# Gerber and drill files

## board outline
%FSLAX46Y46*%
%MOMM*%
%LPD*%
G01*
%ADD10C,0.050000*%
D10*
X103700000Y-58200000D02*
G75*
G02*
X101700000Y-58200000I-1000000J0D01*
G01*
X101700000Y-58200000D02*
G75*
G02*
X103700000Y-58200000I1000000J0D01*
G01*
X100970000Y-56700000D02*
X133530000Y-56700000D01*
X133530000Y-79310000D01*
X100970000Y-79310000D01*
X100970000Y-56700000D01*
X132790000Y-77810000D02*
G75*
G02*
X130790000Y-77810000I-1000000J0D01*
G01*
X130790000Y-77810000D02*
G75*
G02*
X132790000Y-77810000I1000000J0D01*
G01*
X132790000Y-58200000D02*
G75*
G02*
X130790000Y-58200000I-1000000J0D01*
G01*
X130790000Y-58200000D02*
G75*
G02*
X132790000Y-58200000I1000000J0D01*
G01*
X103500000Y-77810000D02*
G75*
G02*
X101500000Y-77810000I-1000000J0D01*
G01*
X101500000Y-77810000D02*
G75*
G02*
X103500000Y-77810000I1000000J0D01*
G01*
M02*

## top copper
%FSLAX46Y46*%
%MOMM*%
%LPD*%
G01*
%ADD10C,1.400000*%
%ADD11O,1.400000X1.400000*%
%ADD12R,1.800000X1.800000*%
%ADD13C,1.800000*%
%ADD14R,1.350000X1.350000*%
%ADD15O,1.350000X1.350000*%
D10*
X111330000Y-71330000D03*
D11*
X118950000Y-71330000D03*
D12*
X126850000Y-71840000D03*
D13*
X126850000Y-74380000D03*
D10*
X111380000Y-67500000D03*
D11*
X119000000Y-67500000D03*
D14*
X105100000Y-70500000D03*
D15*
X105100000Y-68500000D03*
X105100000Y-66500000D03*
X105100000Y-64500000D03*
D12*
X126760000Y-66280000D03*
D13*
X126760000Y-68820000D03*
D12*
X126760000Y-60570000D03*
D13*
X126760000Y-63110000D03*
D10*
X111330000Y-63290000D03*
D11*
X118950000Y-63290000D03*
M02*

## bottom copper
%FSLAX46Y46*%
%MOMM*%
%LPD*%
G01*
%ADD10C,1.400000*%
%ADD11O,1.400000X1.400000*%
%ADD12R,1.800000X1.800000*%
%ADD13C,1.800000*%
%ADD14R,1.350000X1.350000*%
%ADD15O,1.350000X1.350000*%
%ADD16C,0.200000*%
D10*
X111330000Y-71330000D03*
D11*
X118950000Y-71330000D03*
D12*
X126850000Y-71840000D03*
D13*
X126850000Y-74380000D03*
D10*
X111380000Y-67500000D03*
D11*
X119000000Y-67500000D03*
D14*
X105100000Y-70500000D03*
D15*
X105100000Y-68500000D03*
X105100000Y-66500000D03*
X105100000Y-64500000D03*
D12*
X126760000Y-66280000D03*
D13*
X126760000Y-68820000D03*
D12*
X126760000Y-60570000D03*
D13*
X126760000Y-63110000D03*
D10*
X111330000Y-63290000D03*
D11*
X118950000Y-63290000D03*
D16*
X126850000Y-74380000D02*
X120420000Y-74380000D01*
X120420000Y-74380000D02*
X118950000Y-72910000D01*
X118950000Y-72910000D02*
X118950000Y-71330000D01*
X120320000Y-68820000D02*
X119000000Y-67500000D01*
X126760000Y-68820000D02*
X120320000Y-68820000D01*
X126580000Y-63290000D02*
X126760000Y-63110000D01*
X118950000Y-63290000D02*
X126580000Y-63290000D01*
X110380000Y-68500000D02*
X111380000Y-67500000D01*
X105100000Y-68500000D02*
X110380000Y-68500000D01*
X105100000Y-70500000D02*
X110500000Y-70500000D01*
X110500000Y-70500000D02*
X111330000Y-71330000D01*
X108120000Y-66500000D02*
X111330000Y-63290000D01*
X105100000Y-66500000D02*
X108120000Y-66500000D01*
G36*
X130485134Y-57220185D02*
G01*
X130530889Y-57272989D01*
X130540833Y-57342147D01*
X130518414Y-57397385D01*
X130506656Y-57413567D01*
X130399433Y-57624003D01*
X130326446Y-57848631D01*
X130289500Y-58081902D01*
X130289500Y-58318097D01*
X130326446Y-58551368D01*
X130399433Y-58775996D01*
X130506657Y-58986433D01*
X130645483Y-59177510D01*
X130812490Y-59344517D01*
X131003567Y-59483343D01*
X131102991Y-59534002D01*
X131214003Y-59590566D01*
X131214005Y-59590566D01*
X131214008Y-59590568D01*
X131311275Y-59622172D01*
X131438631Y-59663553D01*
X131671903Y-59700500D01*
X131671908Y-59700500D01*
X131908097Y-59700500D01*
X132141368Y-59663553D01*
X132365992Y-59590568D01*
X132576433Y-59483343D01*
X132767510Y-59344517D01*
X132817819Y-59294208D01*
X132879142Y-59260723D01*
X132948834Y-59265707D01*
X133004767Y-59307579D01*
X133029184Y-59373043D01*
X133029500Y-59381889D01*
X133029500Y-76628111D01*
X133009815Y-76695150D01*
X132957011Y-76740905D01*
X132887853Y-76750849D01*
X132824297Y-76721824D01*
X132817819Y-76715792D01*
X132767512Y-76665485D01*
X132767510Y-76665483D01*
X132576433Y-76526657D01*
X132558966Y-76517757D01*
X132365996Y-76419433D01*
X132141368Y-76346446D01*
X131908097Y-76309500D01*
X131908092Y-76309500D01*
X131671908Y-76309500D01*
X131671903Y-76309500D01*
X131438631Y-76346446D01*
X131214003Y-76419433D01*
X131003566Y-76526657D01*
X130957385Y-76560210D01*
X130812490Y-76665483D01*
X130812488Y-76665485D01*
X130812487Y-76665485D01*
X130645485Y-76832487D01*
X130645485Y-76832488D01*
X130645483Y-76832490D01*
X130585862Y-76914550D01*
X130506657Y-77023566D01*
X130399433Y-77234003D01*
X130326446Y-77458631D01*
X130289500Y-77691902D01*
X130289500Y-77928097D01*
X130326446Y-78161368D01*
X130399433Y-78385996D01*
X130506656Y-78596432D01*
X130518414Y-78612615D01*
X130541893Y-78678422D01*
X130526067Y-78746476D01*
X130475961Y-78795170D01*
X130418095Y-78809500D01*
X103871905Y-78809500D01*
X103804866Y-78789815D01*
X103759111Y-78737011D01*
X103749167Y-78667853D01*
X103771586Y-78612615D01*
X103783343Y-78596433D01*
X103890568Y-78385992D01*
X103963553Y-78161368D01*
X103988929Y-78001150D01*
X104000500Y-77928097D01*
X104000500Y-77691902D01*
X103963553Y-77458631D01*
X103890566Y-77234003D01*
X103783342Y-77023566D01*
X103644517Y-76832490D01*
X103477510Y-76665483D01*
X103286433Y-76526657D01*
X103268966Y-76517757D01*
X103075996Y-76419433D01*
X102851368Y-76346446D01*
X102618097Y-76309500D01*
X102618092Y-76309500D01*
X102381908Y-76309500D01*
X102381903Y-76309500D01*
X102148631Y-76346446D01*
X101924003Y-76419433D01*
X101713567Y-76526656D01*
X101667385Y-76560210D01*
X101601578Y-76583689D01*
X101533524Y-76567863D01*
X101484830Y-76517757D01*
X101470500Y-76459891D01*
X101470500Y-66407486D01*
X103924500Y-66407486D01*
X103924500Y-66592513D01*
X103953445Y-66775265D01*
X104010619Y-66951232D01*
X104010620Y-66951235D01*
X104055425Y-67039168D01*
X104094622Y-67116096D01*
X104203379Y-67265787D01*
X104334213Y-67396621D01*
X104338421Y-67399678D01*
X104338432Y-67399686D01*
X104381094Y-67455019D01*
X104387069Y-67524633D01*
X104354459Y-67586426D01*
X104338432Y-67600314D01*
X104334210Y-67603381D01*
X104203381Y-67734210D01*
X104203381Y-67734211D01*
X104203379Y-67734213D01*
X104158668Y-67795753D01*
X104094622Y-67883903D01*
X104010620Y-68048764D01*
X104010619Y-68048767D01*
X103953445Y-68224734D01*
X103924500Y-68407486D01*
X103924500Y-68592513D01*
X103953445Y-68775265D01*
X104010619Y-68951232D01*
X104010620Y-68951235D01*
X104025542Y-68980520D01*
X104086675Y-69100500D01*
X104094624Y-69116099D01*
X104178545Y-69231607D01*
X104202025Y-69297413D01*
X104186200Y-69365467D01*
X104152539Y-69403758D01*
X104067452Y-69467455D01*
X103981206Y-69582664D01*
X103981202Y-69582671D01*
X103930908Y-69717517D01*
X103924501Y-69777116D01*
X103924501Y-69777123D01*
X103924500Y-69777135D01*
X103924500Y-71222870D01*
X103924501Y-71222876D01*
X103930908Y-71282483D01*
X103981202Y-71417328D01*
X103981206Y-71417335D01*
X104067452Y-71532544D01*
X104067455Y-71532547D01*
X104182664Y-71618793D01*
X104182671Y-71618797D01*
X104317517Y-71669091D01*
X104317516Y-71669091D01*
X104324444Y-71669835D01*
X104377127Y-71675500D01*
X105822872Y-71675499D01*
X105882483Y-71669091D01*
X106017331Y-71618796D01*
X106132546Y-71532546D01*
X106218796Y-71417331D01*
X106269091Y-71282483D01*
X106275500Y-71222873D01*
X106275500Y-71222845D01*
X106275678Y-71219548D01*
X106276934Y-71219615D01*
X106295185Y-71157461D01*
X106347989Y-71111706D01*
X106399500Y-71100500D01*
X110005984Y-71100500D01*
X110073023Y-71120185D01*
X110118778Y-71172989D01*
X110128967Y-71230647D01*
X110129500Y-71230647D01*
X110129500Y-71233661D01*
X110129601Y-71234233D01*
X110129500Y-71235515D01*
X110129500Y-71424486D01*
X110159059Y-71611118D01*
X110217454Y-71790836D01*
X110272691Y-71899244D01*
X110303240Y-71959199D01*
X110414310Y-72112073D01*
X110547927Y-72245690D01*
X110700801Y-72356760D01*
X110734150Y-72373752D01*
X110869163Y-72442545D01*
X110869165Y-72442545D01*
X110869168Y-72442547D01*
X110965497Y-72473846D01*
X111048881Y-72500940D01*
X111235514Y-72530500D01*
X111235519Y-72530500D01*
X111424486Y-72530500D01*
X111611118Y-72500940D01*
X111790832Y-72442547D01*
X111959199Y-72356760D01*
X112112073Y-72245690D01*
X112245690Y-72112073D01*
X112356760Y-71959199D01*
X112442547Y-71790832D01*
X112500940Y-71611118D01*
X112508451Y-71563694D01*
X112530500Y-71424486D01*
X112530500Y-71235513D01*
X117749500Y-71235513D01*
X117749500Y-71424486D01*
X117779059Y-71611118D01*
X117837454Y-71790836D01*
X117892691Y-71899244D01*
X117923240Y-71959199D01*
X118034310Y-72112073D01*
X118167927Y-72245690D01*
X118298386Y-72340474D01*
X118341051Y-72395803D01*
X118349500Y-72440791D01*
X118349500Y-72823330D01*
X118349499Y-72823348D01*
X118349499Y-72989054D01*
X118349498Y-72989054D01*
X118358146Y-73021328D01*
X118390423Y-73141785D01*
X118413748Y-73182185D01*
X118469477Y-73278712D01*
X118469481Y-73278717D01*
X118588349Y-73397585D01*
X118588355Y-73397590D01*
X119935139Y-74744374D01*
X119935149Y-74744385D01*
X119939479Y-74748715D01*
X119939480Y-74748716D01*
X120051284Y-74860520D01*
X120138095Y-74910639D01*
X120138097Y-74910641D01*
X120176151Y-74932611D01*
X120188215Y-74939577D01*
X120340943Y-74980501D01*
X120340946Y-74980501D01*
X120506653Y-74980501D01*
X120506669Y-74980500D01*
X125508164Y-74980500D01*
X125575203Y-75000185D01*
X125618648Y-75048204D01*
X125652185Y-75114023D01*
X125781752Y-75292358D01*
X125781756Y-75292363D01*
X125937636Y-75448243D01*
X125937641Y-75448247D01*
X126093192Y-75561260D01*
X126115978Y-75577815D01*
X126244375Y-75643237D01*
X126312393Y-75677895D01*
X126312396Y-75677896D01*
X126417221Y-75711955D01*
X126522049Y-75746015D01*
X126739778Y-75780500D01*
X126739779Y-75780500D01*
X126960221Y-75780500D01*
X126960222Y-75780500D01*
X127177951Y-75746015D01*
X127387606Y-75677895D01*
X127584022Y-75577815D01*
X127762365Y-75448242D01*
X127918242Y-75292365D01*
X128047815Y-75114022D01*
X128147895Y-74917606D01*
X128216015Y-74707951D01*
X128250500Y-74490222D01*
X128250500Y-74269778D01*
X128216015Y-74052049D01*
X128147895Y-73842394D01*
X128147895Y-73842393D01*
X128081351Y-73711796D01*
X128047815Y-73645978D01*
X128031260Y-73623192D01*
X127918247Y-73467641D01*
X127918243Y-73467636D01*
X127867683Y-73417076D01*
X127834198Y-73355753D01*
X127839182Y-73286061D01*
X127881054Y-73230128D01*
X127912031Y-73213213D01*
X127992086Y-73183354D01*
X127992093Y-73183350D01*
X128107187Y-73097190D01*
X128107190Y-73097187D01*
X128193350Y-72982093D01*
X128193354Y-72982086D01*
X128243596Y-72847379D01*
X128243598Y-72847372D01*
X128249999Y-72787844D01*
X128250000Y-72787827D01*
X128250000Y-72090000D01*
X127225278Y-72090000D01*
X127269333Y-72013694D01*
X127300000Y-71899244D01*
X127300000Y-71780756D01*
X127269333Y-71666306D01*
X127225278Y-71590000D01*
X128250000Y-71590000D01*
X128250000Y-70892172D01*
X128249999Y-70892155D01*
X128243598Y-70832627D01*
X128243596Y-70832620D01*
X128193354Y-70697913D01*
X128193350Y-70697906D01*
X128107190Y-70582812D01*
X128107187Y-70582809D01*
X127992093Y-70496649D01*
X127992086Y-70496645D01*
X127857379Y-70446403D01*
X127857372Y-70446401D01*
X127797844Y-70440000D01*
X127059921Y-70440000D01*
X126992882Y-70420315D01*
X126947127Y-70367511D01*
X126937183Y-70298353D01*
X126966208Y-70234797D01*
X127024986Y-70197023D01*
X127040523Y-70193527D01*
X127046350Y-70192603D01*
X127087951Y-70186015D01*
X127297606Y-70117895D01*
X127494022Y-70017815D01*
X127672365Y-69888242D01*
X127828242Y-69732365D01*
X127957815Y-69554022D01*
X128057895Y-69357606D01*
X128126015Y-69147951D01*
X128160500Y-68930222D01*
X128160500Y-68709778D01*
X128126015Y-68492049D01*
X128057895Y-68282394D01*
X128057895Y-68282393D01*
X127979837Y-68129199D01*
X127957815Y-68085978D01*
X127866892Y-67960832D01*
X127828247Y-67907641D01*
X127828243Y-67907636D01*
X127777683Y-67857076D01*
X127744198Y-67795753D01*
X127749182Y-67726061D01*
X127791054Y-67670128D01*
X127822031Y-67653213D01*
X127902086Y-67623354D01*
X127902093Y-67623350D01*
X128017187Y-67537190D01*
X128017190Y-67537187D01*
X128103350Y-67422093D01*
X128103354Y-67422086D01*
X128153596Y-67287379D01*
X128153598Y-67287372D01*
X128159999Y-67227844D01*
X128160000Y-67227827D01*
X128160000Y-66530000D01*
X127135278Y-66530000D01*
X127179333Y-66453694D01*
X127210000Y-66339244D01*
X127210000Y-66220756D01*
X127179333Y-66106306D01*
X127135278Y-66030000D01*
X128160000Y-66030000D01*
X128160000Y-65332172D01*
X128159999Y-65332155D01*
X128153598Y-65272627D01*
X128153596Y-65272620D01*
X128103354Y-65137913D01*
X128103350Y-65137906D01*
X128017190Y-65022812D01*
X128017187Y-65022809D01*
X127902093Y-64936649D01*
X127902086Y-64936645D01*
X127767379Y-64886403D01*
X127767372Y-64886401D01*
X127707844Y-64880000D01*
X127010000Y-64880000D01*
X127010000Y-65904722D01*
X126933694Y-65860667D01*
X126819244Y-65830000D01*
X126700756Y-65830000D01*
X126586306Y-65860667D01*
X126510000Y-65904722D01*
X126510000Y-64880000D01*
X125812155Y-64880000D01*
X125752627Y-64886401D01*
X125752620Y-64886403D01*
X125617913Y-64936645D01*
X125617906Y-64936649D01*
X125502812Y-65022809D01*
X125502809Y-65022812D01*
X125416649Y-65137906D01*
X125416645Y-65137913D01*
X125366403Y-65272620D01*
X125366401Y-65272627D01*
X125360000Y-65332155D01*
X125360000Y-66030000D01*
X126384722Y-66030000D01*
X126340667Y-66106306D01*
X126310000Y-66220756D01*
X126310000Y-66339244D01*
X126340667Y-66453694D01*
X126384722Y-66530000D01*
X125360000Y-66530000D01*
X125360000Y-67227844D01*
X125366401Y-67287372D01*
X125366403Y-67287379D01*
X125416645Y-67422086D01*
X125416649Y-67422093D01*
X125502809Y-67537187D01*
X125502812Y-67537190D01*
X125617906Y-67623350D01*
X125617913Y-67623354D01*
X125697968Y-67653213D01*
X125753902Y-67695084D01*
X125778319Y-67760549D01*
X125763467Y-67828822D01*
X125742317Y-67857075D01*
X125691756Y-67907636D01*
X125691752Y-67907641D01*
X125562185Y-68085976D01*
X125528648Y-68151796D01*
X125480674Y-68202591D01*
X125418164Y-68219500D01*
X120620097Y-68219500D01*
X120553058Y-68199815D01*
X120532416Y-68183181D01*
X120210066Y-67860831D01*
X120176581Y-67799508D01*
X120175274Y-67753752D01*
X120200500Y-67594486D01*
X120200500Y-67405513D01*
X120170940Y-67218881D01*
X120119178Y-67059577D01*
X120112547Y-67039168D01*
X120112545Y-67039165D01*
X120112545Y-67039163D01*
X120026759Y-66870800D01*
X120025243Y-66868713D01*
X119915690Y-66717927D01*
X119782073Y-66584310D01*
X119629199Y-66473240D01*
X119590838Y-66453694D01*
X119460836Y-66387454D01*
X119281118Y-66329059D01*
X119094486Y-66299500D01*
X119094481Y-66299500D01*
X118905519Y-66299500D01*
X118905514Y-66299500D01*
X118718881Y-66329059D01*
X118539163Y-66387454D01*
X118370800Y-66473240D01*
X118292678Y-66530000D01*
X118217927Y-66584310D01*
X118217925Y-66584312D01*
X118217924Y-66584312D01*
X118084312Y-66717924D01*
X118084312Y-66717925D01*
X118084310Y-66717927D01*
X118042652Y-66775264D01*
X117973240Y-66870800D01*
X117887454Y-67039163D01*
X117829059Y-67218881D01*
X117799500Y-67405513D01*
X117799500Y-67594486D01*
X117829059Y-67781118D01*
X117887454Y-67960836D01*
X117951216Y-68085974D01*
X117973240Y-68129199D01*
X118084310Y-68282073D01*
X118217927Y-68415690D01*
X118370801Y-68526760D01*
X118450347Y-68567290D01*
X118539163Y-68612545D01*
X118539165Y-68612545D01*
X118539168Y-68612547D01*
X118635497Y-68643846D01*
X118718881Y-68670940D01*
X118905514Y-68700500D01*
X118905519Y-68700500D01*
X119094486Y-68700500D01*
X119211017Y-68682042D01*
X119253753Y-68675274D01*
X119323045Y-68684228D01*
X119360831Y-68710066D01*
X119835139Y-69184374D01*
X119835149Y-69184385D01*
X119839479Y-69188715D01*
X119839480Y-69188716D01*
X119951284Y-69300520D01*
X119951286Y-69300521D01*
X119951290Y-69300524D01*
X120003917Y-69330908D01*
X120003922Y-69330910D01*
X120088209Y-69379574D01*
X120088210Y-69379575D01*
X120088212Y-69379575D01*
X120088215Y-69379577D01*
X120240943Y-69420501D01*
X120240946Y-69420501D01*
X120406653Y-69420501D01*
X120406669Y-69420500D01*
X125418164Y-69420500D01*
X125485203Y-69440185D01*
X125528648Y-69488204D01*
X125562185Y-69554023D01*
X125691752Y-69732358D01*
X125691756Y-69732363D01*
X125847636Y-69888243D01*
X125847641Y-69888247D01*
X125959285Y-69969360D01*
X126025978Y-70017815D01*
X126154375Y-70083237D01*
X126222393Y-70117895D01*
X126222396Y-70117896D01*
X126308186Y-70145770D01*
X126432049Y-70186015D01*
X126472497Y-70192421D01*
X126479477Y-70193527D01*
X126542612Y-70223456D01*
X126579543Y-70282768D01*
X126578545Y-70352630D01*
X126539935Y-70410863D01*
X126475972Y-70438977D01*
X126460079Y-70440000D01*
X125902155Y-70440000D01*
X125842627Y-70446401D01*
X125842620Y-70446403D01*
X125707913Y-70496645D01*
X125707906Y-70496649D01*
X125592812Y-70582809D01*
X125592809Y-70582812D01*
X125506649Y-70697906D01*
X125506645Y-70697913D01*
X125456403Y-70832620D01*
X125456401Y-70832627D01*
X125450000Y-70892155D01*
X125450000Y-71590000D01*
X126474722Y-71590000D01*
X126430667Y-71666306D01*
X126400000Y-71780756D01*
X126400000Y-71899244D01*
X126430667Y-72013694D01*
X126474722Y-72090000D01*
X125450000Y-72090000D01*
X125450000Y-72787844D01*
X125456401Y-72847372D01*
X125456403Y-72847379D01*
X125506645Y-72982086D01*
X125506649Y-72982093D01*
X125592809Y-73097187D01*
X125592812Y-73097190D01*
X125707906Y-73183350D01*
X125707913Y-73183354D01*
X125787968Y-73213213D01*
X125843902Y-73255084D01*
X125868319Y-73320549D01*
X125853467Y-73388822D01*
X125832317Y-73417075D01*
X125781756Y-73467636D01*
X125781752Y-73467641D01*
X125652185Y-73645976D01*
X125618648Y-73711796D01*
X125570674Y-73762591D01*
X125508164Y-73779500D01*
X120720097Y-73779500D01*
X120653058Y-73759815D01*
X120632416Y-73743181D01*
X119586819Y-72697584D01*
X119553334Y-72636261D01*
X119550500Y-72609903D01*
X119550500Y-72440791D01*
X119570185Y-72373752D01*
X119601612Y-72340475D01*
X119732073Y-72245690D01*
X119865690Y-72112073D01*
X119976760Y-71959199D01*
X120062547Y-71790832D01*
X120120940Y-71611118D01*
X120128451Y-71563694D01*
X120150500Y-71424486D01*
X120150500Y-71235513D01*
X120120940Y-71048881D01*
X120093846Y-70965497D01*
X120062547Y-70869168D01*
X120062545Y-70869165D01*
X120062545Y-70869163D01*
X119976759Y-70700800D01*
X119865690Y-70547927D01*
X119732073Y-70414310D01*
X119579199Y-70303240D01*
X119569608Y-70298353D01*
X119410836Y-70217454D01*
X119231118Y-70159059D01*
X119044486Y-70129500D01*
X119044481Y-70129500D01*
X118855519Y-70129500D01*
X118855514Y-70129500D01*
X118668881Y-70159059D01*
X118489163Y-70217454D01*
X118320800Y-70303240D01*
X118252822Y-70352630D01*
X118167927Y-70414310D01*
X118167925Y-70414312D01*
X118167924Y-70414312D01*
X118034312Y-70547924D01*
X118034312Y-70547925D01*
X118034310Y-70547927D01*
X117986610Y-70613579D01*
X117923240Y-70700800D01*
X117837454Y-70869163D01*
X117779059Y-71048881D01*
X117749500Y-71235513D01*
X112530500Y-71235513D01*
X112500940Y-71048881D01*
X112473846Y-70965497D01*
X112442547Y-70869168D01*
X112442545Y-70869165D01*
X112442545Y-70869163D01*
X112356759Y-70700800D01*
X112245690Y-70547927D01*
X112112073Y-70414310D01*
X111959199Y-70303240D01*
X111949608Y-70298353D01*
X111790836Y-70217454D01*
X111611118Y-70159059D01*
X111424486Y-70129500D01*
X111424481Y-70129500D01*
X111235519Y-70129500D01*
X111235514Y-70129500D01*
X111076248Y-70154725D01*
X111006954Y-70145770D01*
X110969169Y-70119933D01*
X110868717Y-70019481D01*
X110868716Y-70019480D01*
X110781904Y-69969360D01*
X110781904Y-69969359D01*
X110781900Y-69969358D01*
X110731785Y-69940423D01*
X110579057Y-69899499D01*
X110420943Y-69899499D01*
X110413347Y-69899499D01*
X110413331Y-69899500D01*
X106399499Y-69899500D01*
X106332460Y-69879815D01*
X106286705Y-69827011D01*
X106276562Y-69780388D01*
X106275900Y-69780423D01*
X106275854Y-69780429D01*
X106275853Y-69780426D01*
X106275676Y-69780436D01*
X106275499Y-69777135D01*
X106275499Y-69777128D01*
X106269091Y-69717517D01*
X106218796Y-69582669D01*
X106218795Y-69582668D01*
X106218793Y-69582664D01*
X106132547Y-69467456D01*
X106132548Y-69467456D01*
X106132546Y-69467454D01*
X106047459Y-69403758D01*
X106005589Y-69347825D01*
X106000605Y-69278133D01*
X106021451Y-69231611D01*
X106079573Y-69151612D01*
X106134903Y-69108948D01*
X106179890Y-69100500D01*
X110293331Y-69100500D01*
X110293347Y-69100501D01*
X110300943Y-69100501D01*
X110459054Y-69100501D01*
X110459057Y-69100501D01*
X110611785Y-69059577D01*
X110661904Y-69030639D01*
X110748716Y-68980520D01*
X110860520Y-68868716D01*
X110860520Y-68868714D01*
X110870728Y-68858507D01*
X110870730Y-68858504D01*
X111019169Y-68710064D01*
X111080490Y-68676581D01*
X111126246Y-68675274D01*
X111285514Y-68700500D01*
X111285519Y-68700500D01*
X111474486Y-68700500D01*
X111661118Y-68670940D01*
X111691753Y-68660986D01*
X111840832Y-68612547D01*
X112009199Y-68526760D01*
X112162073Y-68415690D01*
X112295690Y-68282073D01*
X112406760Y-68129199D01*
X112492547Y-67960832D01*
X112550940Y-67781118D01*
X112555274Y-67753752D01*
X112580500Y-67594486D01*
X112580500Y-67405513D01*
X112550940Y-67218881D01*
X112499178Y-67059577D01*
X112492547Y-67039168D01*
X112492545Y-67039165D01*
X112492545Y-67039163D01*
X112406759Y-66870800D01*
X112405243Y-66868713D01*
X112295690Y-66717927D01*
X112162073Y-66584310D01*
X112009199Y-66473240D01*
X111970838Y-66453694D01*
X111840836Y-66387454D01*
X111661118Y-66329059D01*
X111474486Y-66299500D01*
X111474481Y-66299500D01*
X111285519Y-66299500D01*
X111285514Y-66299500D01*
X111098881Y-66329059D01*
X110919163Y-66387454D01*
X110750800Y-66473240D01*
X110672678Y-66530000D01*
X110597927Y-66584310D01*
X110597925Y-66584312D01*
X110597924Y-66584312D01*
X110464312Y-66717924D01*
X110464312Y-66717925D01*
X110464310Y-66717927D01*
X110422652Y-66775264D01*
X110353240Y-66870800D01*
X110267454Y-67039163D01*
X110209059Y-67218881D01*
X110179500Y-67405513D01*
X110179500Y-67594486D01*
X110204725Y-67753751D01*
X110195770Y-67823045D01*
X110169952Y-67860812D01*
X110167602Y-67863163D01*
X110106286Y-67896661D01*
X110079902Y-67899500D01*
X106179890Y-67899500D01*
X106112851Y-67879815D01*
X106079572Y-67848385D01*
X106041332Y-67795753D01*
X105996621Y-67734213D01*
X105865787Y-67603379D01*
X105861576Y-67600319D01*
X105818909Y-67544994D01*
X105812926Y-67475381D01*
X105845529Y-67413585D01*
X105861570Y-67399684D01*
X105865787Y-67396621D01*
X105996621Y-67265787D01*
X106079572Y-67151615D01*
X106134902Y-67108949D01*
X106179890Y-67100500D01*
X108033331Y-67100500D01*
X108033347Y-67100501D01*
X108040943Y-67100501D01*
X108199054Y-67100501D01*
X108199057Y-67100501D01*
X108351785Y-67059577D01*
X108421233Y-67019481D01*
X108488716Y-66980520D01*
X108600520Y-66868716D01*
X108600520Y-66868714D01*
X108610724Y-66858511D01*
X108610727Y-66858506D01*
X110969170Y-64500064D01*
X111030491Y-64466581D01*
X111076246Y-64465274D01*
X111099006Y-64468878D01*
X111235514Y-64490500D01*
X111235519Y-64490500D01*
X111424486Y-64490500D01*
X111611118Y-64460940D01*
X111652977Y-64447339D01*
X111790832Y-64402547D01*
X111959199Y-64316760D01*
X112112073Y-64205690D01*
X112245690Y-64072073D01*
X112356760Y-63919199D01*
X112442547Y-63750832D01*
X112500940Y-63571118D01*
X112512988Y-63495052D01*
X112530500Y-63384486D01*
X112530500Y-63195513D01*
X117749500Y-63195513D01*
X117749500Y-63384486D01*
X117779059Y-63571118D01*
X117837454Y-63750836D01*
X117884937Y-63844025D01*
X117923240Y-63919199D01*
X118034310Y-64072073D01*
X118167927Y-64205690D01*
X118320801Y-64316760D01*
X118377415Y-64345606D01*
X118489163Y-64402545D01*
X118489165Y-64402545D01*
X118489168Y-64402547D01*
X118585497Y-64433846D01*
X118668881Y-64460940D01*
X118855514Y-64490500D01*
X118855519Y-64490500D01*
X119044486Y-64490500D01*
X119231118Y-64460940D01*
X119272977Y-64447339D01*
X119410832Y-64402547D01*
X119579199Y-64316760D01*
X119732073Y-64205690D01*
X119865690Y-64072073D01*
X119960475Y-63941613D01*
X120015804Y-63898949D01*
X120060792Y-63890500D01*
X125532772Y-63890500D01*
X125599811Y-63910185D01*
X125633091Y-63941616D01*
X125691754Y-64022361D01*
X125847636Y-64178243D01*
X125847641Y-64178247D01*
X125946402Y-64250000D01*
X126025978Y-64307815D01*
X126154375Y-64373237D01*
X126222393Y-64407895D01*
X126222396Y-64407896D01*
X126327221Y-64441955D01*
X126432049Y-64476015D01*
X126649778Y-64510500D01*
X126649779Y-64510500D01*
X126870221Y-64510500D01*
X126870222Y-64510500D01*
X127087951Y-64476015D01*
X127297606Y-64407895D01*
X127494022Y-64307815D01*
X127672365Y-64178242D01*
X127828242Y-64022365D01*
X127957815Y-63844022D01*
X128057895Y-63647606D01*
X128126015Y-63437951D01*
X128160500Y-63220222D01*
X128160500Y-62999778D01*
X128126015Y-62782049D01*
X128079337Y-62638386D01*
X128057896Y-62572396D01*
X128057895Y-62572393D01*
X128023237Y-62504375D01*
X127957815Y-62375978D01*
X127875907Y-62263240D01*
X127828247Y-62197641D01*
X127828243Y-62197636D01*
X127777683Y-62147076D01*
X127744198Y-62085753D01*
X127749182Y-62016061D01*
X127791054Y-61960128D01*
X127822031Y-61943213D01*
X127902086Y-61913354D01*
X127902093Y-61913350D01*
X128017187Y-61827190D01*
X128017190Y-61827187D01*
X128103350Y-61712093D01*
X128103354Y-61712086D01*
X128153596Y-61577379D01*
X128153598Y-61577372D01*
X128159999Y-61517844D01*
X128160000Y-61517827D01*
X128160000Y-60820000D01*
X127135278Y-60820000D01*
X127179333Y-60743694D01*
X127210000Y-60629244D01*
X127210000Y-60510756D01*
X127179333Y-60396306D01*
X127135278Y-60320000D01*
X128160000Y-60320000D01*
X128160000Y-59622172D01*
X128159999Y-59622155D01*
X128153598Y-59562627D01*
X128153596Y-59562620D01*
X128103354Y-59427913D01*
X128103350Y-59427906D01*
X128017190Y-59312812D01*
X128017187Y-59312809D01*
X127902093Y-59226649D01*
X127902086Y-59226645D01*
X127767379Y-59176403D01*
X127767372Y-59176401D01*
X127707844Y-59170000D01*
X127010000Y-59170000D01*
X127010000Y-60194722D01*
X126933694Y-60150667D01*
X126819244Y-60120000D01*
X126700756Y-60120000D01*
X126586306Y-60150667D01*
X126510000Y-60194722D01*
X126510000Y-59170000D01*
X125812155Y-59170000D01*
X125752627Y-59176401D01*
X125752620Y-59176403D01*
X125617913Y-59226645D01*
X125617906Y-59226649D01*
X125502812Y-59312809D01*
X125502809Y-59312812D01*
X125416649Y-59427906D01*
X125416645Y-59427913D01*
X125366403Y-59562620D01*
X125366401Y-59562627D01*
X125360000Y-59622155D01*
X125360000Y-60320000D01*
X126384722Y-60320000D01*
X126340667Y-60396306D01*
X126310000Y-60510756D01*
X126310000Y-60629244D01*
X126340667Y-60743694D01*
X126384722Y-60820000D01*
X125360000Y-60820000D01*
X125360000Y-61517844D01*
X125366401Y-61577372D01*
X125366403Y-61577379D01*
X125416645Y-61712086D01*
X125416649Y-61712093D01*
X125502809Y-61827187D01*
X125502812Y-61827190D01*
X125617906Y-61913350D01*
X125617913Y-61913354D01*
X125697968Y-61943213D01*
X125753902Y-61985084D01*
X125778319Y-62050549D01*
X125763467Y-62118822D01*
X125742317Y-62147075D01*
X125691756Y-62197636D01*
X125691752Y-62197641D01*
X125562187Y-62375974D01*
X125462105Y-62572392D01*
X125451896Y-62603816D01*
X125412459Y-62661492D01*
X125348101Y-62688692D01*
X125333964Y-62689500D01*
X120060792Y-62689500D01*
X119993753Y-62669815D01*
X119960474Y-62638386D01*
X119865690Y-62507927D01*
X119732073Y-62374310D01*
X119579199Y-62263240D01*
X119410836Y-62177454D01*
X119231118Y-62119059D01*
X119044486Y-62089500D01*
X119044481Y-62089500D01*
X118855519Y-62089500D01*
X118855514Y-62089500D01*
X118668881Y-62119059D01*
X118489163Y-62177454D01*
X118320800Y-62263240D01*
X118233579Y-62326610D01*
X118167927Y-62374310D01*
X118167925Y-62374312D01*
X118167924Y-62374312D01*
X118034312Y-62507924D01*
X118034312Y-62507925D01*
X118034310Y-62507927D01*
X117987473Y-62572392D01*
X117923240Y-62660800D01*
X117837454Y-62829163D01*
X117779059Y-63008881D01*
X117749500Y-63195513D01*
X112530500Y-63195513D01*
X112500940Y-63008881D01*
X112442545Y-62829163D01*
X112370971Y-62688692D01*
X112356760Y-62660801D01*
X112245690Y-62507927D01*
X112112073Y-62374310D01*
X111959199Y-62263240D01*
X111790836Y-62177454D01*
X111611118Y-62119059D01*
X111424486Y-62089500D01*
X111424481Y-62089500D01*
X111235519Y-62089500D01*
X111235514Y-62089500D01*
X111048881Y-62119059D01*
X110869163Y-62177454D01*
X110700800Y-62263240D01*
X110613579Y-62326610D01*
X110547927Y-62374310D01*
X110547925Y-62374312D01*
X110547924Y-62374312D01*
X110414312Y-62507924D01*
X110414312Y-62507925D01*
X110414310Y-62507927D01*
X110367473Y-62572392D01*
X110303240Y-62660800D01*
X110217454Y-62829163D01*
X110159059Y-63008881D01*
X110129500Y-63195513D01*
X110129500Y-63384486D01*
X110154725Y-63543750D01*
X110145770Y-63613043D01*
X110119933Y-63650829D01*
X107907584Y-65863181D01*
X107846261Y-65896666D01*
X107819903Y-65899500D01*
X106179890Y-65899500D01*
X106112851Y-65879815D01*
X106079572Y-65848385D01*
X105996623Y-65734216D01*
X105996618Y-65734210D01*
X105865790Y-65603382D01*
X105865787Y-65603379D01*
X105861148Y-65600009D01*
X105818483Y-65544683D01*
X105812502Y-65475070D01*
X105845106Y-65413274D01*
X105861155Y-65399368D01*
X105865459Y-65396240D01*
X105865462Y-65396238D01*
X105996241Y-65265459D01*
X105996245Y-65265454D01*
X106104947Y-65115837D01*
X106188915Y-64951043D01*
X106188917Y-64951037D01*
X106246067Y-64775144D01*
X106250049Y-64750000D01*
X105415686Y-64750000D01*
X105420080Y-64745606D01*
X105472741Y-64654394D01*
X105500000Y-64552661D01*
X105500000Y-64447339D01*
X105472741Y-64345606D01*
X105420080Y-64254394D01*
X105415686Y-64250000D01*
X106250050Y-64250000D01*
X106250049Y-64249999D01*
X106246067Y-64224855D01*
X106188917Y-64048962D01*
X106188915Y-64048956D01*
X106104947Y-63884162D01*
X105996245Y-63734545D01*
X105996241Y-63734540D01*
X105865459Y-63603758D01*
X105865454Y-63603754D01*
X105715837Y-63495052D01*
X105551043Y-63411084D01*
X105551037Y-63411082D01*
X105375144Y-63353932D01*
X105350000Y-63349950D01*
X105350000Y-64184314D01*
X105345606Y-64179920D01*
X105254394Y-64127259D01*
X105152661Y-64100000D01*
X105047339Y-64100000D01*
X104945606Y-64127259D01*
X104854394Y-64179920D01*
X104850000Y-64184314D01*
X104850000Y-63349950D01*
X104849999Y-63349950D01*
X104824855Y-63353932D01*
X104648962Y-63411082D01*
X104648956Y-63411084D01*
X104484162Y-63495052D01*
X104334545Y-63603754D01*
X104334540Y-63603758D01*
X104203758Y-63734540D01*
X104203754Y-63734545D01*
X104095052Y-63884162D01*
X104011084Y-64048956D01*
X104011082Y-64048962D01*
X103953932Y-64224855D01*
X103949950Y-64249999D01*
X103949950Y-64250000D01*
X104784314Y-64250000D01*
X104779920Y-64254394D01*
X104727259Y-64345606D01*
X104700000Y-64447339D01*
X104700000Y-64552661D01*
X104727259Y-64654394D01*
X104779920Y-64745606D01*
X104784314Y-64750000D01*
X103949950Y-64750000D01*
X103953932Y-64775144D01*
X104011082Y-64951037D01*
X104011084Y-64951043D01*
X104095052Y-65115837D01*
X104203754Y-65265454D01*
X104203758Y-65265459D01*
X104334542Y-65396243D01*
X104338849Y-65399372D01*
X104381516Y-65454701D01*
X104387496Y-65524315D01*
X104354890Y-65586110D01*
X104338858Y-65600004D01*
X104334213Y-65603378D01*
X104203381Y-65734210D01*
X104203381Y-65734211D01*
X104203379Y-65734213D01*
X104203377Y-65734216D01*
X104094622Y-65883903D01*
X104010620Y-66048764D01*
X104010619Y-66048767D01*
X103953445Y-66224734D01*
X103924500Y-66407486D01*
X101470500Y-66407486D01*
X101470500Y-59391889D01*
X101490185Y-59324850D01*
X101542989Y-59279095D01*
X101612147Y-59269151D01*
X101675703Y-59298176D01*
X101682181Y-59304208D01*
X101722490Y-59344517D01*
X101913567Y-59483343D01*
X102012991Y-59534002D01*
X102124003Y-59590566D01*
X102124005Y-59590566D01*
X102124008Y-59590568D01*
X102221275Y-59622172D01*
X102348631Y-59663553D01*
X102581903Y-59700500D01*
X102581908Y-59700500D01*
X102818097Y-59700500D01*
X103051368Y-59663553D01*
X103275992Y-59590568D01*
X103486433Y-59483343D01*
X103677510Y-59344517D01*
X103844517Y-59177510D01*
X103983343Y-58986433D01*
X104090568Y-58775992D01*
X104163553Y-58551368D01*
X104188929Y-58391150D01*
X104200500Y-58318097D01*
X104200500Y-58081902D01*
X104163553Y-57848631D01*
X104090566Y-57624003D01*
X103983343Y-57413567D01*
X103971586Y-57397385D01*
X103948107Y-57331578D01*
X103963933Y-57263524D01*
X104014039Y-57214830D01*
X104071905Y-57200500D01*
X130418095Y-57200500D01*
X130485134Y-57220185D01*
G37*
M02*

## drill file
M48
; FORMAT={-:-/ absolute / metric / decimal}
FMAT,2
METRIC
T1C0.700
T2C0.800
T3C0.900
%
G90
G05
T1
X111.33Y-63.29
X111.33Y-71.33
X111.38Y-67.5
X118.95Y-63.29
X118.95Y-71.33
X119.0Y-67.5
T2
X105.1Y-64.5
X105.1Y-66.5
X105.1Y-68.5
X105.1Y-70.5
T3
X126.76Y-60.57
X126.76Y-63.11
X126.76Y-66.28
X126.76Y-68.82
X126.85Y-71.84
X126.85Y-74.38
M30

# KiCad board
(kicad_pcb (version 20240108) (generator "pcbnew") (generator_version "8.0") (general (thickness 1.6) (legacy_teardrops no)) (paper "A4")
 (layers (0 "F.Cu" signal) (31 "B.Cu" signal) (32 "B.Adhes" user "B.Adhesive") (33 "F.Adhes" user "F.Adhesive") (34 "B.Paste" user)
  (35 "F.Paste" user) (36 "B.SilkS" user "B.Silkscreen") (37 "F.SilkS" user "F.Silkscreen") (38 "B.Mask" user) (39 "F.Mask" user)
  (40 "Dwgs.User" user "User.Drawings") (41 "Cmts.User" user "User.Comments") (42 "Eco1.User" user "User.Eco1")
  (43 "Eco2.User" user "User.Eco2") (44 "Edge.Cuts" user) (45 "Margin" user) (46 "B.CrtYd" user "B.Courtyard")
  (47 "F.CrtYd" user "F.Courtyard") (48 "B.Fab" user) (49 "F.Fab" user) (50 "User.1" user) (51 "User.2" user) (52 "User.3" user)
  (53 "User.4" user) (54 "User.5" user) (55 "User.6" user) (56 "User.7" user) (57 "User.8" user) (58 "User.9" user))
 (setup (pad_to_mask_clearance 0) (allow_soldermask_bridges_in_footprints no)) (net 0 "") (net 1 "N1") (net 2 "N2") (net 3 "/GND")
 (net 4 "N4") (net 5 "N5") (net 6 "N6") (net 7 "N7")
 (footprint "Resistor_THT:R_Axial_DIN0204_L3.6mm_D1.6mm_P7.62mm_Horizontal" (layer "F.Cu") (at 111.33 71.33)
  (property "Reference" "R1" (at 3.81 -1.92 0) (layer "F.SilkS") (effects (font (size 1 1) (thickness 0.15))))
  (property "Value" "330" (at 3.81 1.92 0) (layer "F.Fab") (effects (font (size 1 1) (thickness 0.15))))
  (pad "1" thru_hole circle (at 0 0) (size 1.4 1.4) (drill 0.7) (layers "*.Cu" "*.Mask") (remove_unused_layers no) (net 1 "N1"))
  (pad "2" thru_hole oval (at 7.62 0) (size 1.4 1.4) (drill 0.7) (layers "*.Cu" "*.Mask") (remove_unused_layers no) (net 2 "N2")))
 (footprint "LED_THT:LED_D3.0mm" (layer "F.Cu") (at 126.85 71.84 -90)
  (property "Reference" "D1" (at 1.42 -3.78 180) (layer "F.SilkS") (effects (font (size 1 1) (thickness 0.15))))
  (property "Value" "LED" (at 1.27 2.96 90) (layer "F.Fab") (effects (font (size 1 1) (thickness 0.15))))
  (pad "1" thru_hole rect (at 0 0 270) (size 1.8 1.8) (drill 0.9) (layers "*.Cu" "*.Mask") (remove_unused_layers no) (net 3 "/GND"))
  (pad "2" thru_hole circle (at 2.54 0 270) (size 1.8 1.8) (drill 0.9) (layers "*.Cu" "*.Mask") (remove_unused_layers no) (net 2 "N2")))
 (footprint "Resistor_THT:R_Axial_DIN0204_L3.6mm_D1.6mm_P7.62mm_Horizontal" (layer "F.Cu") (at 111.38 67.5)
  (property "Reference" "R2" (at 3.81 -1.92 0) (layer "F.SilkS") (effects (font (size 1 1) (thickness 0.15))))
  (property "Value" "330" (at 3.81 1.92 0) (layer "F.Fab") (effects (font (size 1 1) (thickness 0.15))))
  (pad "1" thru_hole circle (at 0 0) (size 1.4 1.4) (drill 0.7) (layers "*.Cu" "*.Mask") (remove_unused_layers no) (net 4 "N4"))
  (pad "2" thru_hole oval (at 7.62 0) (size 1.4 1.4) (drill 0.7) (layers "*.Cu" "*.Mask") (remove_unused_layers no) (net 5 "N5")))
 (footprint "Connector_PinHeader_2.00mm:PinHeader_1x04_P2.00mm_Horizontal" (layer "F.Cu") (at 105.1 70.5 180)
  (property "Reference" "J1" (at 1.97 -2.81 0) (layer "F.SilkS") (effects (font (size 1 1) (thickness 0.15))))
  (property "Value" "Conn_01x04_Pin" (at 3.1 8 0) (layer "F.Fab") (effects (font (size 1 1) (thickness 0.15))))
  (pad "1" thru_hole rect (at 0 0 180) (size 1.35 1.35) (drill 0.8) (layers "*.Cu" "*.Mask") (remove_unused_layers no) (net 1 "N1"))
  (pad "2" thru_hole oval (at 0 2 180) (size 1.35 1.35) (drill 0.8) (layers "*.Cu" "*.Mask") (remove_unused_layers no) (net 4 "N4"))
  (pad "3" thru_hole oval (at 0 4 180) (size 1.35 1.35) (drill 0.8) (layers "*.Cu" "*.Mask") (remove_unused_layers no) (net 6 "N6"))
  (pad "4" thru_hole oval (at 0 6 180) (size 1.35 1.35) (drill 0.8) (layers "*.Cu" "*.Mask") (remove_unused_layers no) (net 3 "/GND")))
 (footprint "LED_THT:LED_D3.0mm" (layer "F.Cu") (at 126.76 66.28 -90)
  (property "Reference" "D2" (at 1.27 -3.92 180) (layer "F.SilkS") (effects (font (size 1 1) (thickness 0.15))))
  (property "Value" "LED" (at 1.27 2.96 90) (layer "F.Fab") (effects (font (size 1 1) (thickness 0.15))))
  (pad "1" thru_hole rect (at 0 0 270) (size 1.8 1.8) (drill 0.9) (layers "*.Cu" "*.Mask") (remove_unused_layers no) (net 3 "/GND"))
  (pad "2" thru_hole circle (at 2.54 0 270) (size 1.8 1.8) (drill 0.9) (layers "*.Cu" "*.Mask") (remove_unused_layers no) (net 5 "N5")))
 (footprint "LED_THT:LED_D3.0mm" (layer "F.Cu") (at 126.76 60.57 -90)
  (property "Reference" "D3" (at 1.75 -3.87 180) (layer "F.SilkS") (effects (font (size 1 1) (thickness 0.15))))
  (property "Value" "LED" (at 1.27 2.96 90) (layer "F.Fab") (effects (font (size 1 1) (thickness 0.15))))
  (pad "1" thru_hole rect (at 0 0 270) (size 1.8 1.8) (drill 0.9) (layers "*.Cu" "*.Mask") (remove_unused_layers no) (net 3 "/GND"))
  (pad "2" thru_hole circle (at 2.54 0 270) (size 1.8 1.8) (drill 0.9) (layers "*.Cu" "*.Mask") (remove_unused_layers no) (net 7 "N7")))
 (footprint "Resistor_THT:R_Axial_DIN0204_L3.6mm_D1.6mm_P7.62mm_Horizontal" (layer "F.Cu") (at 111.33 63.29)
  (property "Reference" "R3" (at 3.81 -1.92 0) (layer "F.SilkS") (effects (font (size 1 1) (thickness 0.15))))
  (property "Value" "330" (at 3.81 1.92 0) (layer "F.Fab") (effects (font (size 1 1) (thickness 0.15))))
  (pad "1" thru_hole circle (at 0 0) (size 1.4 1.4) (drill 0.7) (layers "*.Cu" "*.Mask") (remove_unused_layers no) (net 6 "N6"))
  (pad "2" thru_hole oval (at 7.62 0) (size 1.4 1.4) (drill 0.7) (layers "*.Cu" "*.Mask") (remove_unused_layers no) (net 7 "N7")))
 (gr_circle (center 102.7 58.2) (end 103.7 58.2) (stroke (width 0.05) (type default)) (fill none) (layer "Edge.Cuts"))
 (gr_rect (start 100.97 56.7) (end 133.53 79.31) (stroke (width 0.05) (type default)) (fill none) (layer "Edge.Cuts"))
 (gr_circle (center 131.79 77.81) (end 132.79 77.81) (stroke (width 0.05) (type default)) (fill none) (layer "Edge.Cuts"))
 (gr_circle (center 131.79 58.2) (end 132.79 58.2) (stroke (width 0.05) (type default)) (fill none) (layer "Edge.Cuts"))
 (gr_circle (center 102.5 77.81) (end 103.5 77.81) (stroke (width 0.05) (type default)) (fill none) (layer "Edge.Cuts"))
 (segment (start 126.85 74.38) (end 120.42 74.38) (width 0.2) (layer "B.Cu") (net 2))
 (segment (start 120.42 74.38) (end 118.95 72.91) (width 0.2) (layer "B.Cu") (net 2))
 (segment (start 118.95 72.91) (end 118.95 71.33) (width 0.2) (layer "B.Cu") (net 2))
 (segment (start 120.32 68.82) (end 119 67.5) (width 0.2) (layer "B.Cu") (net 5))
 (segment (start 126.76 68.82) (end 120.32 68.82) (width 0.2) (layer "B.Cu") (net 5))
 (segment (start 126.58 63.29) (end 126.76 63.11) (width 0.2) (layer "B.Cu") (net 7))
 (segment (start 118.95 63.29) (end 126.58 63.29) (width 0.2) (layer "B.Cu") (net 7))
 (segment (start 110.38 68.5) (end 111.38 67.5) (width 0.2) (layer "B.Cu") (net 4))
 (segment (start 105.1 68.5) (end 110.38 68.5) (width 0.2) (layer "B.Cu") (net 4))
 (segment (start 105.1 70.5) (end 110.5 70.5) (width 0.2) (layer "B.Cu") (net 1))
 (segment (start 110.5 70.5) (end 111.33 71.33) (width 0.2) (layer "B.Cu") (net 1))
 (segment (start 108.12 66.5) (end 111.33 63.29) (width 0.2) (layer "B.Cu") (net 6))
 (segment (start 105.1 66.5) (end 108.12 66.5) (width 0.2) (layer "B.Cu") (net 6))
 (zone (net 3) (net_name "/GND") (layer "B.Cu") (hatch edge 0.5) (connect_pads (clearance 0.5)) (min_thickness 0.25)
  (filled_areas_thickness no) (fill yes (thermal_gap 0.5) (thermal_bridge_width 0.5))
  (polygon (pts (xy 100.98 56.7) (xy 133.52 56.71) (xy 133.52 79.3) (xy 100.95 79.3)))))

